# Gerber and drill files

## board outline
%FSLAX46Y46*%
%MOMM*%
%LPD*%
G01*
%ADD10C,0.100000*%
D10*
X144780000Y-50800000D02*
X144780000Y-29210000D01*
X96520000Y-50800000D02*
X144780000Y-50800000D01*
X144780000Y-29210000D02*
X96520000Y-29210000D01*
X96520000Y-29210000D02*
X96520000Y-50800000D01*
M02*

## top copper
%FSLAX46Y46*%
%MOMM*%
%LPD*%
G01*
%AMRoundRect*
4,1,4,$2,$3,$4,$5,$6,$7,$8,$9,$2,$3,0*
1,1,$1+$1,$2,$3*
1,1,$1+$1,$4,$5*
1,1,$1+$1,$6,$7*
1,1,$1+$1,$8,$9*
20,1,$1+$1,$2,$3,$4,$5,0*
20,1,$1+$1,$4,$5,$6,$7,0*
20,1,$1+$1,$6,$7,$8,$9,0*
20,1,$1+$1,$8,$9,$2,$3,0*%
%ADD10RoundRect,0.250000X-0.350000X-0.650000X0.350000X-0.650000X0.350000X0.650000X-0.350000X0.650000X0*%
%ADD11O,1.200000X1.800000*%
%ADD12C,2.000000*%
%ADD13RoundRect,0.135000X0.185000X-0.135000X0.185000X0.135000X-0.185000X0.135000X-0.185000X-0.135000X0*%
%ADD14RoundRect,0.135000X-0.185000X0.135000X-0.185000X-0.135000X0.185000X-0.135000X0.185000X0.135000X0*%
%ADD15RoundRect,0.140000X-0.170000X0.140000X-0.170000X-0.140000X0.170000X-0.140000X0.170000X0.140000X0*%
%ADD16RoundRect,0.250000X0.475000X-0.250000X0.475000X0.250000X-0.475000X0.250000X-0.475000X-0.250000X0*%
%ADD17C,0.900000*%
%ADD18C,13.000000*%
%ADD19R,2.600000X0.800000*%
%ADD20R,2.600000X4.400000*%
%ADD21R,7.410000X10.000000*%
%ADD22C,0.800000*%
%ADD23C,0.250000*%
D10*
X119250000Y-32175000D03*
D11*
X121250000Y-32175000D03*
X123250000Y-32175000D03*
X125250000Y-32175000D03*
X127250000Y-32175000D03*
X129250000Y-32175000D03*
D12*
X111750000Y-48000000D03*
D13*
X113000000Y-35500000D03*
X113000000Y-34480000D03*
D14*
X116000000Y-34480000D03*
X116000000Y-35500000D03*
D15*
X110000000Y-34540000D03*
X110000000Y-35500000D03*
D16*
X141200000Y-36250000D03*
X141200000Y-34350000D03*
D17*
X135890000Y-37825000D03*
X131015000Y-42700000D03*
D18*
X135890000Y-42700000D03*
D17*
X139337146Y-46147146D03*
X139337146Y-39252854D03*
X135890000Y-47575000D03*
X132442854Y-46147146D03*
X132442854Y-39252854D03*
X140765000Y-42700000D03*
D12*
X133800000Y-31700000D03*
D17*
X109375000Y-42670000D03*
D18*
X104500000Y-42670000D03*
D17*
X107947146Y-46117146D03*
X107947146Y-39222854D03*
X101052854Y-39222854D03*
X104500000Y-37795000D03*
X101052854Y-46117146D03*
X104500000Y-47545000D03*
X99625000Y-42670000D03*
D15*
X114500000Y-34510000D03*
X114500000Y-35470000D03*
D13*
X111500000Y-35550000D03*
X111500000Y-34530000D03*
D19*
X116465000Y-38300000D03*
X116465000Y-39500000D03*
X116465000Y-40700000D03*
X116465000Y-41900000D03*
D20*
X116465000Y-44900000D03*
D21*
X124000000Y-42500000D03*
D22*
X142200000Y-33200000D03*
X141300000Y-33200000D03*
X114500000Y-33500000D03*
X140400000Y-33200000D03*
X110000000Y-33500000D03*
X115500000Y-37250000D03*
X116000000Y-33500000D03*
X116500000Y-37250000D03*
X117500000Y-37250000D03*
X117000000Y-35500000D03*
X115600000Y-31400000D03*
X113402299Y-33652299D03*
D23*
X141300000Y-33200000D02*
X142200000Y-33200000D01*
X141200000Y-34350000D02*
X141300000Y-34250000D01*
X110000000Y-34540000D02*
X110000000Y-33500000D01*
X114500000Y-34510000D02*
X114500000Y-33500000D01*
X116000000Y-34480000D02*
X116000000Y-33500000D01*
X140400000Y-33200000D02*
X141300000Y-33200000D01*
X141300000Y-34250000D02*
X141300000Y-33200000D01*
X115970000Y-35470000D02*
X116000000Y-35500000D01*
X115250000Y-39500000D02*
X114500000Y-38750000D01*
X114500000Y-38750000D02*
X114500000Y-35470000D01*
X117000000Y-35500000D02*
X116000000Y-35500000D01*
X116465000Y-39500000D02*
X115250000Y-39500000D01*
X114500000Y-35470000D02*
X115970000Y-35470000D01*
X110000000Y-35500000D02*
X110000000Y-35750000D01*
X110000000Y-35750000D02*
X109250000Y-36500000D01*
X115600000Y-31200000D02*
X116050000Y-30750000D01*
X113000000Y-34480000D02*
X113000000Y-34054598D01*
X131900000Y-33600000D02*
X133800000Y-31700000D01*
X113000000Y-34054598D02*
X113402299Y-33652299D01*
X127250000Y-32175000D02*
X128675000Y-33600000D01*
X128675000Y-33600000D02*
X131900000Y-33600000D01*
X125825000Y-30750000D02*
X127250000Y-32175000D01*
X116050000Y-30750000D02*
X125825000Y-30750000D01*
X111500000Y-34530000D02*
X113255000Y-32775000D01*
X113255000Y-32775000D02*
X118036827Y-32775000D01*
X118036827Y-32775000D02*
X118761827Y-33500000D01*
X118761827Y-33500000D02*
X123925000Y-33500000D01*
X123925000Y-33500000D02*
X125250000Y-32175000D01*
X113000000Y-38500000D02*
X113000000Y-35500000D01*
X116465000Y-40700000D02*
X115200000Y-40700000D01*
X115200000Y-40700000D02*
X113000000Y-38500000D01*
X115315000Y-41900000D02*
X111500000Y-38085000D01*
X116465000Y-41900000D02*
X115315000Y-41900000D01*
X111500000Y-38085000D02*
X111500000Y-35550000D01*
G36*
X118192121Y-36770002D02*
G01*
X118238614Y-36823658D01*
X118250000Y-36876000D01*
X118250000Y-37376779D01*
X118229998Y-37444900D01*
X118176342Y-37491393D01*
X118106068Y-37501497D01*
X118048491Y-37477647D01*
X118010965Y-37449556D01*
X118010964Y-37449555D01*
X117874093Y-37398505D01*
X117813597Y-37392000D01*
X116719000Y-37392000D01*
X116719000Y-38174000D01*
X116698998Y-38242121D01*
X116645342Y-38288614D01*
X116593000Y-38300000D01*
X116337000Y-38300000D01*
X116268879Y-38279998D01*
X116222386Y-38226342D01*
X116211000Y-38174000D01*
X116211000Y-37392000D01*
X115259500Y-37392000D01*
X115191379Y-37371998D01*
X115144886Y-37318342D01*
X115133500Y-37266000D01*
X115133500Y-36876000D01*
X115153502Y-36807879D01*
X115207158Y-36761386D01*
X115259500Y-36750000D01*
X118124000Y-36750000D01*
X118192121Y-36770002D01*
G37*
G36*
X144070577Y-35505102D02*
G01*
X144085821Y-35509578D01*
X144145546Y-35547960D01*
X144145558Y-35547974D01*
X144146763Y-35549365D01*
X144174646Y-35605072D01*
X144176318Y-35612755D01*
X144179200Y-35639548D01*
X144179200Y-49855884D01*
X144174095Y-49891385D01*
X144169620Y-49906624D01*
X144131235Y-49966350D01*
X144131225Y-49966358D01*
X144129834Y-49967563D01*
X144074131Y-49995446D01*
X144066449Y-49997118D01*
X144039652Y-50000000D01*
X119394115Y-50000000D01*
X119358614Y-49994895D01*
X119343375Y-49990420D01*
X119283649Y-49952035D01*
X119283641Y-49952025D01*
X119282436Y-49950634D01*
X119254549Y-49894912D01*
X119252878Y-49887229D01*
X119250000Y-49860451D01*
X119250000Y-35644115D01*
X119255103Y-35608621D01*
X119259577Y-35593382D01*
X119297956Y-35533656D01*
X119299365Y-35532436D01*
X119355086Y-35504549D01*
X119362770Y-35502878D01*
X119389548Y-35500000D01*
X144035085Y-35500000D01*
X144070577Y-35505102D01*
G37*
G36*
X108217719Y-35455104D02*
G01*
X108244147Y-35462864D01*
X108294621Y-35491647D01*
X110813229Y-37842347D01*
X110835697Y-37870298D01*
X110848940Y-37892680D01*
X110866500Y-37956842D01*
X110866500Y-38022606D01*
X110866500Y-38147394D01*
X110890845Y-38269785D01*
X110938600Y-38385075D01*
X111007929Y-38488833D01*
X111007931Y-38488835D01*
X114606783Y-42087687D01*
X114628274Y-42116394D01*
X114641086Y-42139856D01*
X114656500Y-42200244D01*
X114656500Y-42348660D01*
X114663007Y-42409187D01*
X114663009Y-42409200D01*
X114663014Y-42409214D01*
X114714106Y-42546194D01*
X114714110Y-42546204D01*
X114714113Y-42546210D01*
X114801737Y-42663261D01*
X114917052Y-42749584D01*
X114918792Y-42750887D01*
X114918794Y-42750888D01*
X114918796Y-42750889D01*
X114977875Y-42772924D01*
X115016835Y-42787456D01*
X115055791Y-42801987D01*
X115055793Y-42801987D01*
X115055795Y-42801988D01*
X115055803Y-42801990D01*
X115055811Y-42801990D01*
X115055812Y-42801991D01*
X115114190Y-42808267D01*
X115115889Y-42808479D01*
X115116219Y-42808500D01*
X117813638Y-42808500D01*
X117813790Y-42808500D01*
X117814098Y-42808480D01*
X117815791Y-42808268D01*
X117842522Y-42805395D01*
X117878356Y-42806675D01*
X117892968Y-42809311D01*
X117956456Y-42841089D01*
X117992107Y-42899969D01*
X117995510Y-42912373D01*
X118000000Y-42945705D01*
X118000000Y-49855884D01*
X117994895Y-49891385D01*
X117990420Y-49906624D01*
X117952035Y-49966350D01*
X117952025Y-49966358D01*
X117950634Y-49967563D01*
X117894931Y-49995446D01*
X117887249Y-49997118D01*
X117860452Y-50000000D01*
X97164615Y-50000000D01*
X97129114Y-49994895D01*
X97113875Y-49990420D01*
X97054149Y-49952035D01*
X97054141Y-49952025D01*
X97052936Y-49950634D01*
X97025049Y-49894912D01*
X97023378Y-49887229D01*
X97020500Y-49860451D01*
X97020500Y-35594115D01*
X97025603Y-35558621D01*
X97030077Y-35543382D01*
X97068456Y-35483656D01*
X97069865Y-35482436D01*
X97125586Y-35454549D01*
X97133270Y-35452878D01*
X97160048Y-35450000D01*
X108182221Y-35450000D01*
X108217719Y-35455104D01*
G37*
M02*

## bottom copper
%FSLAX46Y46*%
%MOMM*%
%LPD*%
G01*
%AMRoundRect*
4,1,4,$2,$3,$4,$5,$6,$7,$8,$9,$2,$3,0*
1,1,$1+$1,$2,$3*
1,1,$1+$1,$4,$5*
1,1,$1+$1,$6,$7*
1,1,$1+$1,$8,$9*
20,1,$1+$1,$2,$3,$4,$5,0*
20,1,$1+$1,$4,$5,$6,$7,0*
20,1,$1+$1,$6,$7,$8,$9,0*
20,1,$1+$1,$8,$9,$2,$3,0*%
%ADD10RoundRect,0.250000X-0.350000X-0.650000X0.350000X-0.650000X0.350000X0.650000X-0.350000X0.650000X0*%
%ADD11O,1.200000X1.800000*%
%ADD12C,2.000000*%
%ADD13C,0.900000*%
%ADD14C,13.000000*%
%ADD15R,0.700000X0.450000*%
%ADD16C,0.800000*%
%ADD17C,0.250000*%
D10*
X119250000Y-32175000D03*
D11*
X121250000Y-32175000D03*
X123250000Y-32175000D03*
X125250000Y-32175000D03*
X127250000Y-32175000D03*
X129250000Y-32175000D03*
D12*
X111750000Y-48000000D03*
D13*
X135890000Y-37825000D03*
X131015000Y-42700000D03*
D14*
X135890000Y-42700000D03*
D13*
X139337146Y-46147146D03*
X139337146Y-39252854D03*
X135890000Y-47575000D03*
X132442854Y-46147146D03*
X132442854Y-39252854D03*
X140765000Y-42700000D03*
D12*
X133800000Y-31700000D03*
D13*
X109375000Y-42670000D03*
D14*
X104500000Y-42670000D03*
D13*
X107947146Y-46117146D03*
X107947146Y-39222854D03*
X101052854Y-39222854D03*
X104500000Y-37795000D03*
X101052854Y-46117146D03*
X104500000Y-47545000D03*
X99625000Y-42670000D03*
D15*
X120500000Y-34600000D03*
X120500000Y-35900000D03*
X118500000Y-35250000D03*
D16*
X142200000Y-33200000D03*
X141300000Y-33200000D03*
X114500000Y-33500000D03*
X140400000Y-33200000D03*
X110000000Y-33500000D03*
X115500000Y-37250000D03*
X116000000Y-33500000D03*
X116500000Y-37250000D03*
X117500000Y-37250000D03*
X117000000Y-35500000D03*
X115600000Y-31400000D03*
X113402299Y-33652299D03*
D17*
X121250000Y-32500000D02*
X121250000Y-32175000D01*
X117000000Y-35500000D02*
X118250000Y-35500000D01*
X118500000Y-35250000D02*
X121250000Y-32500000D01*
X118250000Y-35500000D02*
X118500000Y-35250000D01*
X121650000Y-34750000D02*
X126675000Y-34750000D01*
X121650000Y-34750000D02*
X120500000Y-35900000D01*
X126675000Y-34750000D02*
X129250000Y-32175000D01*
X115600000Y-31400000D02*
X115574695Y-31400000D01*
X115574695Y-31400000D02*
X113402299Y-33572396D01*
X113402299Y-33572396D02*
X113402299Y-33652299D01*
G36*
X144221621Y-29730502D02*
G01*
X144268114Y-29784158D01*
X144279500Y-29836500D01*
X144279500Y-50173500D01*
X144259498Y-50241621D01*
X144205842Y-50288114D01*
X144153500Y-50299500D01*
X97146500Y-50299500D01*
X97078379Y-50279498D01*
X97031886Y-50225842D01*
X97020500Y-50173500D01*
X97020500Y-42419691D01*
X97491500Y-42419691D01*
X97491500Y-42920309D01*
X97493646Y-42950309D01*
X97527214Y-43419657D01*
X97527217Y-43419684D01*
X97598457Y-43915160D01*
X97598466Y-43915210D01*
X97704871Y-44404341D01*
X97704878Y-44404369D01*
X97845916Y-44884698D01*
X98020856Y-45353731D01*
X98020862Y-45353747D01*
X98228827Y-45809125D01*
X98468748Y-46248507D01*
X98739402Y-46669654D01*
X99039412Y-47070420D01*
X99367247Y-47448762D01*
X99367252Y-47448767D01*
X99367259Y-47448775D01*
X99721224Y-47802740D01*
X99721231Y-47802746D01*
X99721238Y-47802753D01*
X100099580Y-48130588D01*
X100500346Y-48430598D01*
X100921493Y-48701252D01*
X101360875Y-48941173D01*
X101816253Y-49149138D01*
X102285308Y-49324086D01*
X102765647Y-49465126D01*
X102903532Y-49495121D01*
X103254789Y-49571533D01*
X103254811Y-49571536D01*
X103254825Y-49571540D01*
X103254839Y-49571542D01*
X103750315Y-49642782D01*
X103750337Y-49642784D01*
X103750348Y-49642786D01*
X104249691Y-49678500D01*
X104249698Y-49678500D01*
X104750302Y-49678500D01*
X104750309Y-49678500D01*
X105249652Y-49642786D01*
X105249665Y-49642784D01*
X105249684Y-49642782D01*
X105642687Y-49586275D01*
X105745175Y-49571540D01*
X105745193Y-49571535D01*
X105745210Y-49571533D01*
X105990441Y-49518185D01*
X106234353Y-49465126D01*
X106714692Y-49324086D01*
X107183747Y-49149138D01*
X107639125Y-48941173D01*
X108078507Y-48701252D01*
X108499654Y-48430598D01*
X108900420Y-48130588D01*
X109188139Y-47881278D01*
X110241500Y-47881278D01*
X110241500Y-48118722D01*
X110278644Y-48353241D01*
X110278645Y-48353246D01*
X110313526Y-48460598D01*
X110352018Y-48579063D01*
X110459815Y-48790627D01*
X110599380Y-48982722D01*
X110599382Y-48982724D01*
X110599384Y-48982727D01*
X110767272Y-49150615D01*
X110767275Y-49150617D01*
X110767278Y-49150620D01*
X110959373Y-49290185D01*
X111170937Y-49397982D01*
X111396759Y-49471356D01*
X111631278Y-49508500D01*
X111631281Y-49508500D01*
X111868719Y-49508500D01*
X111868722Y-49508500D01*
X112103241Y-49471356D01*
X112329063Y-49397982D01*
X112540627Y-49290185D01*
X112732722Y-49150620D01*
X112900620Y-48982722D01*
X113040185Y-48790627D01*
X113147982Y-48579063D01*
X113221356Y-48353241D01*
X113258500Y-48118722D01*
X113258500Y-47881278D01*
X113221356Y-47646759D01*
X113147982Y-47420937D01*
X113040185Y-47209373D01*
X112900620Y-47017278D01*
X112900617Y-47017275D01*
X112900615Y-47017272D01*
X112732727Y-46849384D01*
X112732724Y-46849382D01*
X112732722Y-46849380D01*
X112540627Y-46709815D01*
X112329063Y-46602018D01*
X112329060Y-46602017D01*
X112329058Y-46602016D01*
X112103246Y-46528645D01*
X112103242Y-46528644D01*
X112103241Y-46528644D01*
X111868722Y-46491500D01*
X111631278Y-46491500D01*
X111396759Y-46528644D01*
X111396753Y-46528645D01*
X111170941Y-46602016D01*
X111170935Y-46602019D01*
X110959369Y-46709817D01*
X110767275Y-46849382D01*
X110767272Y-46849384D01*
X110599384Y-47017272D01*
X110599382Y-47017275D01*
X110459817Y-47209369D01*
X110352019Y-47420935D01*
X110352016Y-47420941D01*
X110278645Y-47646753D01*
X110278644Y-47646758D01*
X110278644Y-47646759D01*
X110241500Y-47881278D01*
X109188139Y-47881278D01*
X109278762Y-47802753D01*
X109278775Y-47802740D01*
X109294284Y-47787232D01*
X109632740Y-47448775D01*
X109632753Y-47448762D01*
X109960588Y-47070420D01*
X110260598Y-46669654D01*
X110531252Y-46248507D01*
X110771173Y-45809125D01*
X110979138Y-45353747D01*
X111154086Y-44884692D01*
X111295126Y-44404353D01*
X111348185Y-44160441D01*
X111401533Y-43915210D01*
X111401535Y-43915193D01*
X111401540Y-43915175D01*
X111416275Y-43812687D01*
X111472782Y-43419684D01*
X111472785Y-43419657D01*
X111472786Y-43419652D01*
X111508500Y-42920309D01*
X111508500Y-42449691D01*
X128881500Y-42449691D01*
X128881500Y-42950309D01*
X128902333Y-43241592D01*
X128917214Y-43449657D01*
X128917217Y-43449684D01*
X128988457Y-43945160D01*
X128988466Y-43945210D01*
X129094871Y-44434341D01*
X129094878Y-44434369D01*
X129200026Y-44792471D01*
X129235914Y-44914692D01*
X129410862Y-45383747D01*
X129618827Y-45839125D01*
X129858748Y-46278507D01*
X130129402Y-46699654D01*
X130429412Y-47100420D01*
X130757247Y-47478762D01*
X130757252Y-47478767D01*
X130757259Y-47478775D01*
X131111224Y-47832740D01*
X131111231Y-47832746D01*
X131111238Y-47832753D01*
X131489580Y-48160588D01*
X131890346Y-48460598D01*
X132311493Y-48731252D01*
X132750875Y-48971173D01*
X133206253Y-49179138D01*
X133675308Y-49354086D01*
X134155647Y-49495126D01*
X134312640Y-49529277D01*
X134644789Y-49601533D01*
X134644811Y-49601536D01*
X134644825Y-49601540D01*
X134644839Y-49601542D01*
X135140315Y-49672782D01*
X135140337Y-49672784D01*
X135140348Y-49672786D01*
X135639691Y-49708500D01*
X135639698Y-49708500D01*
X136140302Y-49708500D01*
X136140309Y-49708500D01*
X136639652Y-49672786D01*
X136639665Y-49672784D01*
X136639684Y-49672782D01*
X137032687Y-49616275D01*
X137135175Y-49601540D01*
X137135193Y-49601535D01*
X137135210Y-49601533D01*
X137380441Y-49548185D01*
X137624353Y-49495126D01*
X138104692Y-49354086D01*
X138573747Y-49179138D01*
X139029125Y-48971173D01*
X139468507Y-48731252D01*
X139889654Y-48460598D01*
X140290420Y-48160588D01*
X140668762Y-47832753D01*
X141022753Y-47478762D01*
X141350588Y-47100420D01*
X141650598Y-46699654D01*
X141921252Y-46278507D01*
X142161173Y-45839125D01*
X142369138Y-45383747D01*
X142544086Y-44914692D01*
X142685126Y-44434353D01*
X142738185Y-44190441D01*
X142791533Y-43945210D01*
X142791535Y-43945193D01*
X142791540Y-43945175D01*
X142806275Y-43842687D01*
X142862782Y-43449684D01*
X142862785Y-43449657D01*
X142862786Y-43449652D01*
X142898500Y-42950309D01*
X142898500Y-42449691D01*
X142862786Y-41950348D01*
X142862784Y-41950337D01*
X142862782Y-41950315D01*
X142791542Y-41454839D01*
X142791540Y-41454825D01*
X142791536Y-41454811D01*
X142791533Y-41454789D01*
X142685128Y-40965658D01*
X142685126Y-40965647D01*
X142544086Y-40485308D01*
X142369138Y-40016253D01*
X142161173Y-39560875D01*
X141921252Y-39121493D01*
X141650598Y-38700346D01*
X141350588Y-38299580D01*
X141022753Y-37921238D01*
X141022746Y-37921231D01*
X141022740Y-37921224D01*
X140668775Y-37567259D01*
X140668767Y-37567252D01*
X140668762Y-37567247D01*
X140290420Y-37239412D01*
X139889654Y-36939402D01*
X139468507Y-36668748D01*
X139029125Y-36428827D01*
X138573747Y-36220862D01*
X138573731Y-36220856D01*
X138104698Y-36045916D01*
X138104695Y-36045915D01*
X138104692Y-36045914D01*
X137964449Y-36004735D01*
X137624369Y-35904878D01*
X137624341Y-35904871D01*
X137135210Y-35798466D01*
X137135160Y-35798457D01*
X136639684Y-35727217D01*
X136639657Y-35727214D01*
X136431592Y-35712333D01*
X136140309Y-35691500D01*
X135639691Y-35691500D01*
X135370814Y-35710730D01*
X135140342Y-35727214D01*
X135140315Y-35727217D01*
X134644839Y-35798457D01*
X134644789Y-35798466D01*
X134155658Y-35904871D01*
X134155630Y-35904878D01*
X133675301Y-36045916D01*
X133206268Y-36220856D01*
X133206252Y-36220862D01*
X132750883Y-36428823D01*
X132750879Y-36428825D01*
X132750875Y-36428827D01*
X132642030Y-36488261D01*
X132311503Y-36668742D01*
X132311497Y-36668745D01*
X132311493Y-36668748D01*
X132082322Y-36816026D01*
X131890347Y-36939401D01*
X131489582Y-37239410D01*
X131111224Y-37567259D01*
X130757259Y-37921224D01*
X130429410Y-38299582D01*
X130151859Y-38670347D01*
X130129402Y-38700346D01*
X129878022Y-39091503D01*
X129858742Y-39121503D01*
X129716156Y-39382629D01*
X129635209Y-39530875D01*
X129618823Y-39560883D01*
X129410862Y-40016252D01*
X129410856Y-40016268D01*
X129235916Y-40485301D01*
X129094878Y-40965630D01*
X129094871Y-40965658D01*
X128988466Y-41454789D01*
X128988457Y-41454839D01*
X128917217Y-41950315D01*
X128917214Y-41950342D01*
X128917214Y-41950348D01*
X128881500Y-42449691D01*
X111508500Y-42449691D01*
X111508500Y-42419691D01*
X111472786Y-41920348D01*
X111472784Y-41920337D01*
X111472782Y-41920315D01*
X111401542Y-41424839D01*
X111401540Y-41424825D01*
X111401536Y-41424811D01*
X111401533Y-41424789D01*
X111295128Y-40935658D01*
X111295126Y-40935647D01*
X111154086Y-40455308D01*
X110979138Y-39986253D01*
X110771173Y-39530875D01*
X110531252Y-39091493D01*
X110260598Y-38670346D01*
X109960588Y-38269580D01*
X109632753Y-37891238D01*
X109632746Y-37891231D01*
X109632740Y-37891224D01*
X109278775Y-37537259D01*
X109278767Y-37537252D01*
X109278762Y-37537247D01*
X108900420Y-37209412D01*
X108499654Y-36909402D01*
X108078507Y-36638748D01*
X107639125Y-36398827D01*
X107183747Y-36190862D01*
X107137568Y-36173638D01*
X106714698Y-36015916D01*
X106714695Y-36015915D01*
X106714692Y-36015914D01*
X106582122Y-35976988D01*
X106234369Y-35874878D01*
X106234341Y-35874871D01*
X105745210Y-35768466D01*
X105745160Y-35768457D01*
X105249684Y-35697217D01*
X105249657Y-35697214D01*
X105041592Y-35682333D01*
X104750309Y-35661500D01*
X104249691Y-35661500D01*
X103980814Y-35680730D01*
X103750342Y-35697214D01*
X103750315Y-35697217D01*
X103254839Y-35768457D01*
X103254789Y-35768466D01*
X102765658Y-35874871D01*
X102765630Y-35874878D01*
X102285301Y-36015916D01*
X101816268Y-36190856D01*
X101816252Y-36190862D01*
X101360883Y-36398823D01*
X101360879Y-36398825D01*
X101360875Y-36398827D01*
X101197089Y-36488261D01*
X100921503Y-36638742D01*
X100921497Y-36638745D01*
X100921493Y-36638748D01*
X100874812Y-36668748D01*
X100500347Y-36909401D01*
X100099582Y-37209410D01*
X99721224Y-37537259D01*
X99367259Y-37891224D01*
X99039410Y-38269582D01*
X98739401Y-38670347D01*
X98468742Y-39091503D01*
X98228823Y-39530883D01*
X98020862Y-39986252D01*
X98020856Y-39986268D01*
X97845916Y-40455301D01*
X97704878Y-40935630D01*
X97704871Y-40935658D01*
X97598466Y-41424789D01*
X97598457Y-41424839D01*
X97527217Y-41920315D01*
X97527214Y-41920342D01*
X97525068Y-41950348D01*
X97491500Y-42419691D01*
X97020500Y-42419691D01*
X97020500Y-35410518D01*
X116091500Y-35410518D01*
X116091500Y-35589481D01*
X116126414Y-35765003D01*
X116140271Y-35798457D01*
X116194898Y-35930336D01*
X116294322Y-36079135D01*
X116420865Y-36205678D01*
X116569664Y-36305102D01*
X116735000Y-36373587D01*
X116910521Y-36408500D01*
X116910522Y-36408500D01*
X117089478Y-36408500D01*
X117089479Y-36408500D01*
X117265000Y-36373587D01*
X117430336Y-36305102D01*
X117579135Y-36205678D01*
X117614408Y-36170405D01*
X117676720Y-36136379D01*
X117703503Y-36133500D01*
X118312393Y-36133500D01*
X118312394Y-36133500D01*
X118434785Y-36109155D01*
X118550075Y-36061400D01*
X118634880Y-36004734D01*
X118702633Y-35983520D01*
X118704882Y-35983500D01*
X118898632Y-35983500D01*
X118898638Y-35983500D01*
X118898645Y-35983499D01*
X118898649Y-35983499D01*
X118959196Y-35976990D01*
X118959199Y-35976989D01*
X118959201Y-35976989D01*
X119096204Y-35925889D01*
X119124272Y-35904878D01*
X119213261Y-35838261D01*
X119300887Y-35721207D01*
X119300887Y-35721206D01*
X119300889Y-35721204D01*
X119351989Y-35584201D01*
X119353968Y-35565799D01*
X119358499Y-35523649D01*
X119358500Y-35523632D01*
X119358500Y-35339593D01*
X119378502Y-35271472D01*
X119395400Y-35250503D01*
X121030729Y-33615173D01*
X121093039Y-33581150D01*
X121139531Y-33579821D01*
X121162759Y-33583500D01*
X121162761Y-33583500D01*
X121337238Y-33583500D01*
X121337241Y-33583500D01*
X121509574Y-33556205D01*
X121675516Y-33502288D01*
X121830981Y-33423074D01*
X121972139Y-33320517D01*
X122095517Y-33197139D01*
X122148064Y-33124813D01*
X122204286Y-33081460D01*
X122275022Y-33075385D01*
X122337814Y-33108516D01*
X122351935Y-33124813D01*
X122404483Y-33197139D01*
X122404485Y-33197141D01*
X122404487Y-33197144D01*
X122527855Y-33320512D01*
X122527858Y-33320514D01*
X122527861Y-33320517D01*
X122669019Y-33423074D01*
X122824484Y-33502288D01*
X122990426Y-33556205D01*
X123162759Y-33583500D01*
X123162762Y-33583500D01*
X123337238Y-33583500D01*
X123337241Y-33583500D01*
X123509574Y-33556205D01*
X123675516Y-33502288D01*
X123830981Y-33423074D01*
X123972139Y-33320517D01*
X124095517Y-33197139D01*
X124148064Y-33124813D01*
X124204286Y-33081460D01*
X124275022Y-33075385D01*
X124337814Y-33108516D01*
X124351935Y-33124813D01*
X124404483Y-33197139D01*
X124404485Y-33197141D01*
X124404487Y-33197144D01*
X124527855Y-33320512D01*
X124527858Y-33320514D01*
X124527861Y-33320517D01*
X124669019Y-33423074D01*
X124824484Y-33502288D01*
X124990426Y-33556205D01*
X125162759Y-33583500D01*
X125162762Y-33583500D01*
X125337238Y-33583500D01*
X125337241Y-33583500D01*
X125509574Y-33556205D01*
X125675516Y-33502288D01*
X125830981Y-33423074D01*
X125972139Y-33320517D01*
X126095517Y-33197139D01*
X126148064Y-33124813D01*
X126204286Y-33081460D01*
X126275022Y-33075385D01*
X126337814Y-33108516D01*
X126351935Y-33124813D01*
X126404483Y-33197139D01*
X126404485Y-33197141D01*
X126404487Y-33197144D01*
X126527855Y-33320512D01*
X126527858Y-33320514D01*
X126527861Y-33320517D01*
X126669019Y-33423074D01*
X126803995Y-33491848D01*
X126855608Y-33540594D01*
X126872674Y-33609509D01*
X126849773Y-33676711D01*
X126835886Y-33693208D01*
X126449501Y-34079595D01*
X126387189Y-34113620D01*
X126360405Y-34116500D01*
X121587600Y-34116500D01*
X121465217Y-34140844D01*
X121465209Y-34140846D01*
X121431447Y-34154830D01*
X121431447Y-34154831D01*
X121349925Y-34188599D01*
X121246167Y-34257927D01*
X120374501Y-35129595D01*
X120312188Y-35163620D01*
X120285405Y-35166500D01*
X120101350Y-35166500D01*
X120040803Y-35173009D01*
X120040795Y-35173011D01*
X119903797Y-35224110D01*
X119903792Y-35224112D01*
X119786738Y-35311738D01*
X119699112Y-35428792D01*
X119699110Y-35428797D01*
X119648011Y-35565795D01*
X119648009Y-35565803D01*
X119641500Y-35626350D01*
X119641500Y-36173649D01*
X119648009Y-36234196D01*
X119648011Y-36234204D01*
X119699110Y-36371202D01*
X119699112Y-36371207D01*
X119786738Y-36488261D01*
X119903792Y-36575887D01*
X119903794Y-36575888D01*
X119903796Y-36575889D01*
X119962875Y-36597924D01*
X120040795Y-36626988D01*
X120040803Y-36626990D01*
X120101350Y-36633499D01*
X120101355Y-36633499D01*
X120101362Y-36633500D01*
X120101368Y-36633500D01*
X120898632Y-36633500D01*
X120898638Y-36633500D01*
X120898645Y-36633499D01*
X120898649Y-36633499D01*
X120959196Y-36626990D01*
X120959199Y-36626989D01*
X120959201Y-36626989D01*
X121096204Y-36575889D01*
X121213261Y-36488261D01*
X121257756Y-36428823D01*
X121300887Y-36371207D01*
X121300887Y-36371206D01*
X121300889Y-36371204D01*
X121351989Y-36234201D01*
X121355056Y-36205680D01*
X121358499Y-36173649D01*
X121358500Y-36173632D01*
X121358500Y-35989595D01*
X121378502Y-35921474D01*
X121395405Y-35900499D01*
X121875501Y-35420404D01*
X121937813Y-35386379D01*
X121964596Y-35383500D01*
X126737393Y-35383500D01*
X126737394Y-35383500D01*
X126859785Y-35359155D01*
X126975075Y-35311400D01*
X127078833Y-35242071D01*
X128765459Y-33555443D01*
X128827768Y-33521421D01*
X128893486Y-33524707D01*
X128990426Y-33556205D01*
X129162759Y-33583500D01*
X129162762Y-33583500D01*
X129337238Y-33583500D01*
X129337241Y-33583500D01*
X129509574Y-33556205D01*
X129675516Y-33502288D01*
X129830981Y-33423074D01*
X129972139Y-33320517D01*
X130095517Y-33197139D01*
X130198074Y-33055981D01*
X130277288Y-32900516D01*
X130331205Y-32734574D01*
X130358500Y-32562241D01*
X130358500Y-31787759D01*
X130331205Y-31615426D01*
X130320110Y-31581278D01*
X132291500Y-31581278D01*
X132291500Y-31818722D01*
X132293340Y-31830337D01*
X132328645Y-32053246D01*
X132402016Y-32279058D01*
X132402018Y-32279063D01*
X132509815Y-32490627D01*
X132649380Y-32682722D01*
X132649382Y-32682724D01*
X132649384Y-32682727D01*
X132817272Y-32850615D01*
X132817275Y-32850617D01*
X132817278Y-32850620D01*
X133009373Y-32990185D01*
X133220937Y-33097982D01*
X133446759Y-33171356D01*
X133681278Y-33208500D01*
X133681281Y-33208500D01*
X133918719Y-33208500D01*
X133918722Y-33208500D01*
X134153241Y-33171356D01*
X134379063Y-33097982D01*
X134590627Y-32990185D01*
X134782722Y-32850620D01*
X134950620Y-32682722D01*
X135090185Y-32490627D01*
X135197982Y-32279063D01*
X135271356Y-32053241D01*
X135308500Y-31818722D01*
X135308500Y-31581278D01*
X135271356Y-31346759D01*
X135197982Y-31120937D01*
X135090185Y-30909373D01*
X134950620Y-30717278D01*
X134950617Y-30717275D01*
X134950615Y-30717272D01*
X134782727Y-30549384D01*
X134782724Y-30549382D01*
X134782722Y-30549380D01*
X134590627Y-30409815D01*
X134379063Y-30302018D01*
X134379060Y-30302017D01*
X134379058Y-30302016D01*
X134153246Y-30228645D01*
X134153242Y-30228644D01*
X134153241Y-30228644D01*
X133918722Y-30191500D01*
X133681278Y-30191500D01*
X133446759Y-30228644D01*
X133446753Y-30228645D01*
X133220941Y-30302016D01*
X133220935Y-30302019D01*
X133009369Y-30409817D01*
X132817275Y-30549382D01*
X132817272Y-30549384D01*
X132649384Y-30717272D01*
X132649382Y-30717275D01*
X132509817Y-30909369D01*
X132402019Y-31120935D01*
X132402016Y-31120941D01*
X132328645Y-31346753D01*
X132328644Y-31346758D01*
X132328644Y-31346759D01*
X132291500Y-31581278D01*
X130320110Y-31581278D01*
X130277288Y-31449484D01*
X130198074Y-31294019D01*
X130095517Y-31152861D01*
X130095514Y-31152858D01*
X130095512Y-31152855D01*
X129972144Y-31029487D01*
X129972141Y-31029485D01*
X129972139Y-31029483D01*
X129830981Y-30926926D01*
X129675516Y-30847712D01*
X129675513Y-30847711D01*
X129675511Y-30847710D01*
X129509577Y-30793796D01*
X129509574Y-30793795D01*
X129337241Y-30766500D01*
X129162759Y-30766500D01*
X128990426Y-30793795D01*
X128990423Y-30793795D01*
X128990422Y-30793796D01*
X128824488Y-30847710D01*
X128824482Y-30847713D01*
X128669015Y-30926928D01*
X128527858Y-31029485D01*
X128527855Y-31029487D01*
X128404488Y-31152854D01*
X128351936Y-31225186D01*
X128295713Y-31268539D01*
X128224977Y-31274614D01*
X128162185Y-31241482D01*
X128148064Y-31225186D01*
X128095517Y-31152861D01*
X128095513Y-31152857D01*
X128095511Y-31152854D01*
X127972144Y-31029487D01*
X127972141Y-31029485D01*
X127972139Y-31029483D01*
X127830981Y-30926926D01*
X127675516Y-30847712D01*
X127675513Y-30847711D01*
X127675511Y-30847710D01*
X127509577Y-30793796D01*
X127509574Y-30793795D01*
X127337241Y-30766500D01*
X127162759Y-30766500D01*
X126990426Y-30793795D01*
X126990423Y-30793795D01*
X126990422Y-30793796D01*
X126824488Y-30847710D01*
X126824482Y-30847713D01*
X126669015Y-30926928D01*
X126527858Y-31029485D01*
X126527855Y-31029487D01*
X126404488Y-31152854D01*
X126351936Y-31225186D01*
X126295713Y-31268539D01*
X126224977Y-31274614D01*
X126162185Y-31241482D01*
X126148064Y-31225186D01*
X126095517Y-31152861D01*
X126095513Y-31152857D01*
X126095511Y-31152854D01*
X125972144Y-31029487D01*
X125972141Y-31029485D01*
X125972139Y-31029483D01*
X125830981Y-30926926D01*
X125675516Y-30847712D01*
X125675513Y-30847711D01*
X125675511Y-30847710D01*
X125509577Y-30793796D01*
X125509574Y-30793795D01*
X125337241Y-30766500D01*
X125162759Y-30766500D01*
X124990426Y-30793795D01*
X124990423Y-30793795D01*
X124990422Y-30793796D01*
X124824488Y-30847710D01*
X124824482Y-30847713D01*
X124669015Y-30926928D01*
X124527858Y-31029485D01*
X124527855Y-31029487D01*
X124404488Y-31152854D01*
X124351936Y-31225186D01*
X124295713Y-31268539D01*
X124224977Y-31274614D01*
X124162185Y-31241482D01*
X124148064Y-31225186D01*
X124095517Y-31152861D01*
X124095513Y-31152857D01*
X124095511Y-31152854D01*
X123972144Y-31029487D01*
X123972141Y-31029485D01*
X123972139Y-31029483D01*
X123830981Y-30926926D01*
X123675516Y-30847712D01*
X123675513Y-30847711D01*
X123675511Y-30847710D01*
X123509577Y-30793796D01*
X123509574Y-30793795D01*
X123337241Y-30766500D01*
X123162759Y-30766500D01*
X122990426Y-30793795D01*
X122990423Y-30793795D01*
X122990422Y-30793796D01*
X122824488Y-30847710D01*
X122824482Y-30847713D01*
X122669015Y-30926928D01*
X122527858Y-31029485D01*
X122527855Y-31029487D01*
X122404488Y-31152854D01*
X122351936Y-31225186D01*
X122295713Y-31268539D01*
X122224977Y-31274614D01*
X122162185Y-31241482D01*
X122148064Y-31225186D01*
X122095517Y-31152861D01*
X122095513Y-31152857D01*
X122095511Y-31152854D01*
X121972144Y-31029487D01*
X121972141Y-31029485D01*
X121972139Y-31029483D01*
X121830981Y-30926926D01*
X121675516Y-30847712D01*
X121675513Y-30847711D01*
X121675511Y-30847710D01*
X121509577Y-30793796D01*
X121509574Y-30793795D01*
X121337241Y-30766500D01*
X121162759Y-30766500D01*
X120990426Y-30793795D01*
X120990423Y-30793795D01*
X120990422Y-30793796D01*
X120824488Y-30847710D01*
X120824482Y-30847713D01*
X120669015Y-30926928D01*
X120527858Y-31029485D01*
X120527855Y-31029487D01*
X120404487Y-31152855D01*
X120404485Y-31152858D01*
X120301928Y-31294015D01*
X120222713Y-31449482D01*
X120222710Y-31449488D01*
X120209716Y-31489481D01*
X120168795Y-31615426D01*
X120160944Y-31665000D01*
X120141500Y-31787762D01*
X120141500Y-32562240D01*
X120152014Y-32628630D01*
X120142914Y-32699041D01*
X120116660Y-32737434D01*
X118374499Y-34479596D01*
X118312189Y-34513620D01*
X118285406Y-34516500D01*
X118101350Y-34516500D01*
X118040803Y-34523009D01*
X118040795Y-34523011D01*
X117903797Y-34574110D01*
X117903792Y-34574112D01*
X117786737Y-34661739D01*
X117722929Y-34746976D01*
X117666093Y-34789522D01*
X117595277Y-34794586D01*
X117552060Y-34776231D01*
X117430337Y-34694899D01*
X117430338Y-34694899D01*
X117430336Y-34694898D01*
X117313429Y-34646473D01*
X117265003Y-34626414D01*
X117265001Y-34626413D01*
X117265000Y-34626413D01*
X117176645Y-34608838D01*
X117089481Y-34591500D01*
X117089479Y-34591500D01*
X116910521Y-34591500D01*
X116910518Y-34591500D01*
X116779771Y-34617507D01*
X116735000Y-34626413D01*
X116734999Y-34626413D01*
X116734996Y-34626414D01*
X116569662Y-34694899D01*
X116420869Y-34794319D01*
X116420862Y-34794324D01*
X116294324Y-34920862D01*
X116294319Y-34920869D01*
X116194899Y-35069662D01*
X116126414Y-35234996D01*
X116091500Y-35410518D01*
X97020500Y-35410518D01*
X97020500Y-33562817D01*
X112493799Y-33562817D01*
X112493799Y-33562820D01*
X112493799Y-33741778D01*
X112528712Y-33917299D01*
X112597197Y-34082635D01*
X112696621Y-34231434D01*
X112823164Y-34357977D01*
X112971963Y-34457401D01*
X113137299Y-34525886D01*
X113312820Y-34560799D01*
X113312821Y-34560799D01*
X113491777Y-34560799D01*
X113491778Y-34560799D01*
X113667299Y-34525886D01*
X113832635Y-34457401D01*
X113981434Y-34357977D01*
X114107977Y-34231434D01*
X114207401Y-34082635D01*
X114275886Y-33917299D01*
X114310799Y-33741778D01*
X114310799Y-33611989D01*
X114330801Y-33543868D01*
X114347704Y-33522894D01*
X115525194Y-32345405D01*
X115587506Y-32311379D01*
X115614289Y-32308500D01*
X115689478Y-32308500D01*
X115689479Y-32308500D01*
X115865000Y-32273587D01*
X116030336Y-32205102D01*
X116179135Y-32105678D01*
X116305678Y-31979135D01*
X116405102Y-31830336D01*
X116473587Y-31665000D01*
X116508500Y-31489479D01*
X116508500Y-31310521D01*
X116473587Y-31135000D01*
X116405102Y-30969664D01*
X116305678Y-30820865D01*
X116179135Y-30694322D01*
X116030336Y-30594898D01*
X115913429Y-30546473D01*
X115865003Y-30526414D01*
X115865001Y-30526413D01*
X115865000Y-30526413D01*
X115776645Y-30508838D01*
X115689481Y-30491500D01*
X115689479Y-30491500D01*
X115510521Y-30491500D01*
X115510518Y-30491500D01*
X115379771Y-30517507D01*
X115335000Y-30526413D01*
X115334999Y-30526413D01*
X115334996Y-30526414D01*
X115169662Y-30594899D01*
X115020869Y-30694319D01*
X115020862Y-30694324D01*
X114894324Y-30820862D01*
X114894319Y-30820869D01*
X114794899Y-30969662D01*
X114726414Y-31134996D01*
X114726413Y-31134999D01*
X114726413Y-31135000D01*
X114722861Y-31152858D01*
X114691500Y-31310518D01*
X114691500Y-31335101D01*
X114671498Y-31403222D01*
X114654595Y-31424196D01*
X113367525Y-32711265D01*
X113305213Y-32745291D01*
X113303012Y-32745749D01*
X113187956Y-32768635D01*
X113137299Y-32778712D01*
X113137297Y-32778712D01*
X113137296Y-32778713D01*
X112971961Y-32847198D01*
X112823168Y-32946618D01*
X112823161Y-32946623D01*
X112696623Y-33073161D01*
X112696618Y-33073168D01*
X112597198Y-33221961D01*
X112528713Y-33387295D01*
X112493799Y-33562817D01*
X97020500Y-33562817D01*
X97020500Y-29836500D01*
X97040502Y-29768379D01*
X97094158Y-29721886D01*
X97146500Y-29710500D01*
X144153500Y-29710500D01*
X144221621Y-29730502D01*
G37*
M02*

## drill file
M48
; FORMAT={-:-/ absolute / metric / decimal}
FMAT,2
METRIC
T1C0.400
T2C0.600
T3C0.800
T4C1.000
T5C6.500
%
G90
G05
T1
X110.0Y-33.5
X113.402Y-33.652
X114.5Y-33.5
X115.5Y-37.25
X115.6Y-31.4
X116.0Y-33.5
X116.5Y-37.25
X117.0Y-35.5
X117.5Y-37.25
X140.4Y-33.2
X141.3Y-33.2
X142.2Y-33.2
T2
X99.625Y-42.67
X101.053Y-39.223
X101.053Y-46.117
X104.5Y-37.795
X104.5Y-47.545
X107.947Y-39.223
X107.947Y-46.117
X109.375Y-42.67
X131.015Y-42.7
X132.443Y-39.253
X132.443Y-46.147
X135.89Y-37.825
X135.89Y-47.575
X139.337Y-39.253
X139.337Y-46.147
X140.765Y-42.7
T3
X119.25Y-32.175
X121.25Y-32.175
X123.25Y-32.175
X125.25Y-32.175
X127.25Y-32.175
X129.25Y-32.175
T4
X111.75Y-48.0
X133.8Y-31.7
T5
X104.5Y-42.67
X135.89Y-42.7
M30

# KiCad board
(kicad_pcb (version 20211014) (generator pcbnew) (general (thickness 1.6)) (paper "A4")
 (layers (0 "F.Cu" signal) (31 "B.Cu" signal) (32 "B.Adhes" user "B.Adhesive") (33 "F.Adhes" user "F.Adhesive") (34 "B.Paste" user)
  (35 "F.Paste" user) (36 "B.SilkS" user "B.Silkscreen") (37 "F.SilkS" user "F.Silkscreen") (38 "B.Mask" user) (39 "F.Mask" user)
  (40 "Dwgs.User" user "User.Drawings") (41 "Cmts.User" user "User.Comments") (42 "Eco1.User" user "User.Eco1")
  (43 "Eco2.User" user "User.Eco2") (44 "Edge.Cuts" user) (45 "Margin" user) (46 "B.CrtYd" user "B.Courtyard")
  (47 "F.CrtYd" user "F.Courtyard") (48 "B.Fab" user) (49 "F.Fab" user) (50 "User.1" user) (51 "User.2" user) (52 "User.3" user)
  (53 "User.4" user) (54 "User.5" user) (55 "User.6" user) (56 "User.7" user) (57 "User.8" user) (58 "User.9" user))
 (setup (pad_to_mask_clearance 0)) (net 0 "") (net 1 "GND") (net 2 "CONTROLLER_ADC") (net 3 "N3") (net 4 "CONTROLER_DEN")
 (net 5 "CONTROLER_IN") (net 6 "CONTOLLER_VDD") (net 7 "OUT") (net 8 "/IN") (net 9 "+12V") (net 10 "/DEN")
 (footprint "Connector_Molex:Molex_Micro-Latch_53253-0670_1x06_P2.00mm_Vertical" (layer "F.Cu") (at 119.25 32.175)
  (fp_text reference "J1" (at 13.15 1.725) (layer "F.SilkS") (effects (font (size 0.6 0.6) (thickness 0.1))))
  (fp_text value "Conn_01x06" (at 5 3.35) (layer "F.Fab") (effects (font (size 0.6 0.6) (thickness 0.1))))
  (pad "1" thru_hole roundrect (at 0 0) (size 1.2 1.8) (drill 0.8) (layers *.Cu *.Mask) (roundrect_rratio 0.208333) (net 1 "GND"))
  (pad "2" thru_hole oval (at 2 0) (size 1.2 1.8) (drill 0.8) (layers *.Cu *.Mask) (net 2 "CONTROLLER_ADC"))
  (pad "3" thru_hole oval (at 4 0) (size 1.2 1.8) (drill 0.8) (layers *.Cu *.Mask) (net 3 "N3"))
  (pad "4" thru_hole oval (at 6 0) (size 1.2 1.8) (drill 0.8) (layers *.Cu *.Mask) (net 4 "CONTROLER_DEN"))
  (pad "5" thru_hole oval (at 8 0) (size 1.2 1.8) (drill 0.8) (layers *.Cu *.Mask) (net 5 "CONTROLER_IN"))
  (pad "6" thru_hole oval (at 10 0) (size 1.2 1.8) (drill 0.8) (layers *.Cu *.Mask) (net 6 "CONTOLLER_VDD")))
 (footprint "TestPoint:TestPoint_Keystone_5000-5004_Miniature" (layer "F.Cu") (at 111.75 48)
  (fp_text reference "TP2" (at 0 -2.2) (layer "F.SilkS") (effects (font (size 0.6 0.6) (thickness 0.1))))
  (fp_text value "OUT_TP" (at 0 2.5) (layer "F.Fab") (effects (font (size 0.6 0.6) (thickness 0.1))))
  (pad "1" thru_hole circle (at 0 0) (size 2 2) (drill 1) (layers *.Cu *.Mask) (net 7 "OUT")))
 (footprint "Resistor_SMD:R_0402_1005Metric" (layer "F.Cu") (at 113 34.99 90)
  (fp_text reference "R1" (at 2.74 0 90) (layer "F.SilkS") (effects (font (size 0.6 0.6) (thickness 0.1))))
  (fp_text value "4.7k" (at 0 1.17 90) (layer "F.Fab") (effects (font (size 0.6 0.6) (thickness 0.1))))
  (pad "1" smd roundrect (at -0.51 0 90) (size 0.54 0.64) (layers "F.Cu" "F.Paste" "F.Mask") (roundrect_rratio 0.25) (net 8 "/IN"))
  (pad "2" smd roundrect (at 0.51 0 90) (size 0.54 0.64) (layers "F.Cu" "F.Paste" "F.Mask") (roundrect_rratio 0.25) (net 5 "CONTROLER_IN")))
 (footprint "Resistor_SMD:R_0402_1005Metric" (layer "F.Cu") (at 116 34.99 -90)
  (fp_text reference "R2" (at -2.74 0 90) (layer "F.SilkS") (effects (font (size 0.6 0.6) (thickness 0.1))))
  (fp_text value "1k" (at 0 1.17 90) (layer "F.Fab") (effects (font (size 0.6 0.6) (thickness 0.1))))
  (pad "1" smd roundrect (at -0.51 0 270) (size 0.54 0.64) (layers "F.Cu" "F.Paste" "F.Mask") (roundrect_rratio 0.25) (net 1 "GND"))
  (pad "2" smd roundrect (at 0.51 0 270) (size 0.54 0.64) (layers "F.Cu" "F.Paste" "F.Mask") (roundrect_rratio 0.25)
   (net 2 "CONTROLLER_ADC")))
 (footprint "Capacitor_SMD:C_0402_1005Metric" (layer "F.Cu") (at 110 35.02 -90)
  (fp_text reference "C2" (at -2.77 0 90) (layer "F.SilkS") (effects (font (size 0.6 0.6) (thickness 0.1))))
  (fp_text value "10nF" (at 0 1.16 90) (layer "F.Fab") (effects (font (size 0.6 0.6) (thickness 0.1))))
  (pad "1" smd roundrect (at -0.48 0 270) (size 0.56 0.62) (layers "F.Cu" "F.Paste" "F.Mask") (roundrect_rratio 0.25) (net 1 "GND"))
  (pad "2" smd roundrect (at 0.48 0 270) (size 0.56 0.62) (layers "F.Cu" "F.Paste" "F.Mask") (roundrect_rratio 0.25) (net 7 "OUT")))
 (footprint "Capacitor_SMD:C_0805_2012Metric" (layer "F.Cu") (at 141.2 35.3 90)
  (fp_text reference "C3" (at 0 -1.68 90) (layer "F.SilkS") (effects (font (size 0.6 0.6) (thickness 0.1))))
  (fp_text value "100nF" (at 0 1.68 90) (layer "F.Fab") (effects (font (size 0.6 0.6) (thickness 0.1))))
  (pad "1" smd roundrect (at -0.95 0 90) (size 1 1.45) (layers "F.Cu" "F.Paste" "F.Mask") (roundrect_rratio 0.25) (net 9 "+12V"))
  (pad "2" smd roundrect (at 0.95 0 90) (size 1 1.45) (layers "F.Cu" "F.Paste" "F.Mask") (roundrect_rratio 0.25) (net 1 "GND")))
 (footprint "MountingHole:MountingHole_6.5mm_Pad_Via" (layer "F.Cu") (at 135.89 42.7)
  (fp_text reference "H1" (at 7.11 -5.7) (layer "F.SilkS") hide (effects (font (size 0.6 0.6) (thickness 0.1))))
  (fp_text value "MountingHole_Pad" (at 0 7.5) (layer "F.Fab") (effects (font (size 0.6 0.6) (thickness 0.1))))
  (pad "1" thru_hole circle (at 0 -4.875) (size 0.9 0.9) (drill 0.6) (layers *.Cu *.Mask) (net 9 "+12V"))
  (pad "1" thru_hole circle (at -4.875 0) (size 0.9 0.9) (drill 0.6) (layers *.Cu *.Mask) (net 9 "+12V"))
  (pad "1" thru_hole circle (at 0 0) (size 13 13) (drill 6.5) (layers *.Cu *.Mask) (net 9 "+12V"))
  (pad "1" thru_hole circle (at 3.447146 3.447146) (size 0.9 0.9) (drill 0.6) (layers *.Cu *.Mask) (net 9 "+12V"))
  (pad "1" thru_hole circle (at 3.447146 -3.447146) (size 0.9 0.9) (drill 0.6) (layers *.Cu *.Mask) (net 9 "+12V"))
  (pad "1" thru_hole circle (at 0 4.875) (size 0.9 0.9) (drill 0.6) (layers *.Cu *.Mask) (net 9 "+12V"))
  (pad "1" thru_hole circle (at -3.447146 3.447146) (size 0.9 0.9) (drill 0.6) (layers *.Cu *.Mask) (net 9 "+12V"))
  (pad "1" thru_hole circle (at -3.447146 -3.447146) (size 0.9 0.9) (drill 0.6) (layers *.Cu *.Mask) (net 9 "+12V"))
  (pad "1" thru_hole circle (at 4.875 0) (size 0.9 0.9) (drill 0.6) (layers *.Cu *.Mask) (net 9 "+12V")))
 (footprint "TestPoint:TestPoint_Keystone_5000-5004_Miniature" (layer "F.Cu") (at 133.8 31.7)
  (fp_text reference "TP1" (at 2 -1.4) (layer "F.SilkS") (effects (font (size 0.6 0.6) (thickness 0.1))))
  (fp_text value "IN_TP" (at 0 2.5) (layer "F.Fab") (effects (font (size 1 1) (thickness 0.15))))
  (pad "1" thru_hole circle (at 0 0) (size 2 2) (drill 1) (layers *.Cu *.Mask) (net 5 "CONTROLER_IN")))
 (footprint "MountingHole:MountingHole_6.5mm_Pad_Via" (layer "F.Cu") (at 104.5 42.67)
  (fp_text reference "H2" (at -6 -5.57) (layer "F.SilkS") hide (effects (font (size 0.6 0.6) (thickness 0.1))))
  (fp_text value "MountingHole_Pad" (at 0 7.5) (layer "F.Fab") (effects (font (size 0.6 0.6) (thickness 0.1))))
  (pad "1" thru_hole circle (at 4.875 0) (size 0.9 0.9) (drill 0.6) (layers *.Cu *.Mask) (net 7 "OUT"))
  (pad "1" thru_hole circle (at 0 0) (size 13 13) (drill 6.5) (layers *.Cu *.Mask) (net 7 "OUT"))
  (pad "1" thru_hole circle (at 3.447146 3.447146) (size 0.9 0.9) (drill 0.6) (layers *.Cu *.Mask) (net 7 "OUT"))
  (pad "1" thru_hole circle (at 3.447146 -3.447146) (size 0.9 0.9) (drill 0.6) (layers *.Cu *.Mask) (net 7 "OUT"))
  (pad "1" thru_hole circle (at -3.447146 -3.447146) (size 0.9 0.9) (drill 0.6) (layers *.Cu *.Mask) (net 7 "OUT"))
  (pad "1" thru_hole circle (at 0 -4.875) (size 0.9 0.9) (drill 0.6) (layers *.Cu *.Mask) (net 7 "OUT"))
  (pad "1" thru_hole circle (at -3.447146 3.447146) (size 0.9 0.9) (drill 0.6) (layers *.Cu *.Mask) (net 7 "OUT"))
  (pad "1" thru_hole circle (at 0 4.875) (size 0.9 0.9) (drill 0.6) (layers *.Cu *.Mask) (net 7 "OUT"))
  (pad "1" thru_hole circle (at -4.875 0) (size 0.9 0.9) (drill 0.6) (layers *.Cu *.Mask) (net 7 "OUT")))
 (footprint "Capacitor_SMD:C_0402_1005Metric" (layer "F.Cu") (at 114.5 34.99 -90)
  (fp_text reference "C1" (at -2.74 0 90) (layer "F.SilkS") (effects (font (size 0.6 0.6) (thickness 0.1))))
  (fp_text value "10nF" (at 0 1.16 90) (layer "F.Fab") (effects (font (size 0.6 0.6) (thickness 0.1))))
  (pad "1" smd roundrect (at -0.48 0 270) (size 0.56 0.62) (layers "F.Cu" "F.Paste" "F.Mask") (roundrect_rratio 0.25) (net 1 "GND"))
  (pad "2" smd roundrect (at 0.48 0 270) (size 0.56 0.62) (layers "F.Cu" "F.Paste" "F.Mask") (roundrect_rratio 0.25)
   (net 2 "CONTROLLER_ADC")))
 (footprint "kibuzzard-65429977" (layer "F.Cu") (at 104.4 34.3)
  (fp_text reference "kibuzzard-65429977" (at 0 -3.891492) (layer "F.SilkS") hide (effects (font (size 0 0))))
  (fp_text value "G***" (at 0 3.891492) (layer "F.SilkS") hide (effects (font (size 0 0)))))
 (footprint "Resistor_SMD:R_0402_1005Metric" (layer "F.Cu") (at 111.5 35.04 90)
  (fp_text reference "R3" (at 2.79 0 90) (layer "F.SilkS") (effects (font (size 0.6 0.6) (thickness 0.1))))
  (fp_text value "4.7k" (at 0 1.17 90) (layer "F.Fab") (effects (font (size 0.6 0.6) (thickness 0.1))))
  (pad "1" smd roundrect (at -0.51 0 90) (size 0.54 0.64) (layers "F.Cu" "F.Paste" "F.Mask") (roundrect_rratio 0.25) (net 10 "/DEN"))
  (pad "2" smd roundrect (at 0.51 0 90) (size 0.54 0.64) (layers "F.Cu" "F.Paste" "F.Mask") (roundrect_rratio 0.25) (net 4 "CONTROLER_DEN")))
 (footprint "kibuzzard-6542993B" (layer "F.Cu") (at 136 34.4)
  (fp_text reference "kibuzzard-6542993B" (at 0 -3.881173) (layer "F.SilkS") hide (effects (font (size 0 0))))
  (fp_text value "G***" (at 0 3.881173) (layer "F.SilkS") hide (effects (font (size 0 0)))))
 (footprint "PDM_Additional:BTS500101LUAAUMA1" (layer "F.Cu") (at 121.435 42.5 -90)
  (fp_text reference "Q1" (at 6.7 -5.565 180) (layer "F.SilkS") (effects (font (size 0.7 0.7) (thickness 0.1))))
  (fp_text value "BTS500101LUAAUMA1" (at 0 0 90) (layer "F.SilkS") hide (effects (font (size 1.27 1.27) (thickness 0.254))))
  (pad "1" smd rect (at -4.2 4.97 270) (size 0.8 2.6) (layers "F.Cu" "F.Paste" "F.Mask") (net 1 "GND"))
  (pad "2" smd rect (at -3 4.97 270) (size 0.8 2.6) (layers "F.Cu" "F.Paste" "F.Mask") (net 2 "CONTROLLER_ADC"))
  (pad "3" smd rect (at -1.8 4.97 270) (size 0.8 2.6) (layers "F.Cu" "F.Paste" "F.Mask") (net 8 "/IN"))
  (pad "4" smd rect (at -0.6 4.97 270) (size 0.8 2.6) (layers "F.Cu" "F.Paste" "F.Mask") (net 10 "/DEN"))
  (pad "5" smd rect (at 2.4 4.97) (size 2.6 4.4) (layers "F.Cu" "F.Paste" "F.Mask") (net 7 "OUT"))
  (pad "9" smd rect (at 0 -2.565) (size 7.41 10) (layers "F.Cu" "F.Paste" "F.Mask") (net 9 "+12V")))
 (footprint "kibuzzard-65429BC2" (layer "B.Cu") (at 104.14 31.75 180)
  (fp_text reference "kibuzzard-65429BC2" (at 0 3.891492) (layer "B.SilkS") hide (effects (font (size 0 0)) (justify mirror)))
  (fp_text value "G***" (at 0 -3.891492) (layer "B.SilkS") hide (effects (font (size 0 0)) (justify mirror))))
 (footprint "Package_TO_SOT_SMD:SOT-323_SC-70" (layer "B.Cu") (at 119.5 35.25 180)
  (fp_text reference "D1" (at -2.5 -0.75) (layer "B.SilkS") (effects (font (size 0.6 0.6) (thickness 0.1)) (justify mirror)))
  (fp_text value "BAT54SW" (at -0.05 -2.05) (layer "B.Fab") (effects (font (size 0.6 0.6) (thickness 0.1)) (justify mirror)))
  (pad "1" smd rect (at -1 0.65 270) (size 0.45 0.7) (layers "B.Cu" "B.Paste" "B.Mask") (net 1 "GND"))
  (pad "2" smd rect (at -1 -0.65 270) (size 0.45 0.7) (layers "B.Cu" "B.Paste" "B.Mask") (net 6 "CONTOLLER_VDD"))
  (pad "3" smd rect (at 1 0 270) (size 0.45 0.7) (layers "B.Cu" "B.Paste" "B.Mask") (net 2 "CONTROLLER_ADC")))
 (gr_line (start 144.78 50.8) (end 144.78 29.21) (layer "Edge.Cuts") (width 0.1))
 (gr_line (start 96.52 50.8) (end 144.78 50.8) (layer "Edge.Cuts") (width 0.1))
 (gr_line (start 144.78 29.21) (end 96.52 29.21) (layer "Edge.Cuts") (width 0.1))
 (gr_line (start 96.52 29.21) (end 96.52 50.8) (layer "Edge.Cuts") (width 0.1))
 (segment (start 141.3 33.2) (end 142.2 33.2) (width 0.25) (layer "F.Cu") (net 1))
 (segment (start 141.2 34.35) (end 141.3 34.25) (width 0.25) (layer "F.Cu") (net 1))
 (segment (start 110 34.54) (end 110 33.5) (width 0.25) (layer "F.Cu") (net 1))
 (segment (start 114.5 34.51) (end 114.5 33.5) (width 0.25) (layer "F.Cu") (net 1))
 (segment (start 116 34.48) (end 116 33.5) (width 0.25) (layer "F.Cu") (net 1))
 (segment (start 140.4 33.2) (end 141.3 33.2) (width 0.25) (layer "F.Cu") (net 1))
 (segment (start 141.3 34.25) (end 141.3 33.2) (width 0.25) (layer "F.Cu") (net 1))
 (via (at 142.2 33.2) (size 0.8) (drill 0.4) (layers "F.Cu" "B.Cu") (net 1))
 (via (at 141.3 33.2) (size 0.8) (drill 0.4) (layers "F.Cu" "B.Cu") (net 1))
 (via (at 114.5 33.5) (size 0.8) (drill 0.4) (layers "F.Cu" "B.Cu") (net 1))
 (via (at 140.4 33.2) (size 0.8) (drill 0.4) (layers "F.Cu" "B.Cu") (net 1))
 (via (at 110 33.5) (size 0.8) (drill 0.4) (layers "F.Cu" "B.Cu") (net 1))
 (via (at 115.5 37.25) (size 0.8) (drill 0.4) (layers "F.Cu" "B.Cu") (free) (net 1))
 (via (at 116 33.5) (size 0.8) (drill 0.4) (layers "F.Cu" "B.Cu") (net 1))
 (via (at 116.5 37.25) (size 0.8) (drill 0.4) (layers "F.Cu" "B.Cu") (free) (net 1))
 (via (at 117.5 37.25) (size 0.8) (drill 0.4) (layers "F.Cu" "B.Cu") (free) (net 1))
 (segment (start 115.97 35.47) (end 116 35.5) (width 0.25) (layer "F.Cu") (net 2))
 (segment (start 115.25 39.5) (end 114.5 38.75) (width 0.25) (layer "F.Cu") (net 2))
 (segment (start 114.5 38.75) (end 114.5 35.47) (width 0.25) (layer "F.Cu") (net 2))
 (segment (start 117 35.5) (end 116 35.5) (width 0.25) (layer "F.Cu") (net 2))
 (segment (start 116.465 39.5) (end 115.25 39.5) (width 0.25) (layer "F.Cu") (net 2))
 (segment (start 114.5 35.47) (end 115.97 35.47) (width 0.25) (layer "F.Cu") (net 2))
 (via (at 117 35.5) (size 0.8) (drill 0.4) (layers "F.Cu" "B.Cu") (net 2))
 (segment (start 121.25 32.5) (end 121.25 32.175) (width 0.25) (layer "B.Cu") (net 2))
 (segment (start 117 35.5) (end 118.25 35.5) (width 0.25) (layer "B.Cu") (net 2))
 (segment (start 118.5 35.25) (end 121.25 32.5) (width 0.25) (layer "B.Cu") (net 2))
 (segment (start 118.25 35.5) (end 118.5 35.25) (width 0.25) (layer "B.Cu") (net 2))
 (segment (start 110 35.5) (end 110 35.75) (width 0.25) (layer "F.Cu") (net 7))
 (segment (start 110 35.75) (end 109.25 36.5) (width 0.25) (layer "F.Cu") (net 7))
 (segment (start 121.65 34.75) (end 126.675 34.75) (width 0.25) (layer "B.Cu") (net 6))
 (segment (start 121.65 34.75) (end 120.5 35.9) (width 0.25) (layer "B.Cu") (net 6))
 (segment (start 126.675 34.75) (end 129.25 32.175) (width 0.25) (layer "B.Cu") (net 6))
 (segment (start 115.6 31.2) (end 116.05 30.75) (width 0.25) (layer "F.Cu") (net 5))
 (segment (start 113 34.48) (end 113 34.054598) (width 0.25) (layer "F.Cu") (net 5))
 (segment (start 131.9 33.6) (end 133.8 31.7) (width 0.25) (layer "F.Cu") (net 5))
 (segment (start 113 34.054598) (end 113.402299 33.652299) (width 0.25) (layer "F.Cu") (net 5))
 (segment (start 127.25 32.175) (end 128.675 33.6) (width 0.25) (layer "F.Cu") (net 5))
 (segment (start 128.675 33.6) (end 131.9 33.6) (width 0.25) (layer "F.Cu") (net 5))
 (segment (start 125.825 30.75) (end 127.25 32.175) (width 0.25) (layer "F.Cu") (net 5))
 (segment (start 116.05 30.75) (end 125.825 30.75) (width 0.25) (layer "F.Cu") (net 5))
 (via (at 115.6 31.4) (size 0.8) (drill 0.4) (layers "F.Cu" "B.Cu") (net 5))
 (via (at 113.402299 33.652299) (size 0.8) (drill 0.4) (layers "F.Cu" "B.Cu") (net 5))
 (segment (start 115.6 31.4) (end 115.574695 31.4) (width 0.25) (layer "B.Cu") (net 5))
 (segment (start 115.574695 31.4) (end 113.402299 33.572396) (width 0.25) (layer "B.Cu") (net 5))
 (segment (start 113.402299 33.572396) (end 113.402299 33.652299) (width 0.25) (layer "B.Cu") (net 5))
 (segment (start 111.5 34.53) (end 113.255 32.775) (width 0.25) (layer "F.Cu") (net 4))
 (segment (start 113.255 32.775) (end 118.036827 32.775) (width 0.25) (layer "F.Cu") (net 4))
 (segment (start 118.036827 32.775) (end 118.761827 33.5) (width 0.25) (layer "F.Cu") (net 4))
 (segment (start 118.761827 33.5) (end 123.925 33.5) (width 0.25) (layer "F.Cu") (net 4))
 (segment (start 123.925 33.5) (end 125.25 32.175) (width 0.25) (layer "F.Cu") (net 4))
 (segment (start 113 38.5) (end 113 35.5) (width 0.25) (layer "F.Cu") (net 8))
 (segment (start 116.465 40.7) (end 115.2 40.7) (width 0.25) (layer "F.Cu") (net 8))
 (segment (start 115.2 40.7) (end 113 38.5) (width 0.25) (layer "F.Cu") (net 8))
 (segment (start 115.315 41.9) (end 111.5 38.085) (width 0.25) (layer "F.Cu") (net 10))
 (segment (start 116.465 41.9) (end 115.315 41.9) (width 0.25) (layer "F.Cu") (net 10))
 (segment (start 111.5 38.085) (end 111.5 35.55) (width 0.25) (layer "F.Cu") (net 10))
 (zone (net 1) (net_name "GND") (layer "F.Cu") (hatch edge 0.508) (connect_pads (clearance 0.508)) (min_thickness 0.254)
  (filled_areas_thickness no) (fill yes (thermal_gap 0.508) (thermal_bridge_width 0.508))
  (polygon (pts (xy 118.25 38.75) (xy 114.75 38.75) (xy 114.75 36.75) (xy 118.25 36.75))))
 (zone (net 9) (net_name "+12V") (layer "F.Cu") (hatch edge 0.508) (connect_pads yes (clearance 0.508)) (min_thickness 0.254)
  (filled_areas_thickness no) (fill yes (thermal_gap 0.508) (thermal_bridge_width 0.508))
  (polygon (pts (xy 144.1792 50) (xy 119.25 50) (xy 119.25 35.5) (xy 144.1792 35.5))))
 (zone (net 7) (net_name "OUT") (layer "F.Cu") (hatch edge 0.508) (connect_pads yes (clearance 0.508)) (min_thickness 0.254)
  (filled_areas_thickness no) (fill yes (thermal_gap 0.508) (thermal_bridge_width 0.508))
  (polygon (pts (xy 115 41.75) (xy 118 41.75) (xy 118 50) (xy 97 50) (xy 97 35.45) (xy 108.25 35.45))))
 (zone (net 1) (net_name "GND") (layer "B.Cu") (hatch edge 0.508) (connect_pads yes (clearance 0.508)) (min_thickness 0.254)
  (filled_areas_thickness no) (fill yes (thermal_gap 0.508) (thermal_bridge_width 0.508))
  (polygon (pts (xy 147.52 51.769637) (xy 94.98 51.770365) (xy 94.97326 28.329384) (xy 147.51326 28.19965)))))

